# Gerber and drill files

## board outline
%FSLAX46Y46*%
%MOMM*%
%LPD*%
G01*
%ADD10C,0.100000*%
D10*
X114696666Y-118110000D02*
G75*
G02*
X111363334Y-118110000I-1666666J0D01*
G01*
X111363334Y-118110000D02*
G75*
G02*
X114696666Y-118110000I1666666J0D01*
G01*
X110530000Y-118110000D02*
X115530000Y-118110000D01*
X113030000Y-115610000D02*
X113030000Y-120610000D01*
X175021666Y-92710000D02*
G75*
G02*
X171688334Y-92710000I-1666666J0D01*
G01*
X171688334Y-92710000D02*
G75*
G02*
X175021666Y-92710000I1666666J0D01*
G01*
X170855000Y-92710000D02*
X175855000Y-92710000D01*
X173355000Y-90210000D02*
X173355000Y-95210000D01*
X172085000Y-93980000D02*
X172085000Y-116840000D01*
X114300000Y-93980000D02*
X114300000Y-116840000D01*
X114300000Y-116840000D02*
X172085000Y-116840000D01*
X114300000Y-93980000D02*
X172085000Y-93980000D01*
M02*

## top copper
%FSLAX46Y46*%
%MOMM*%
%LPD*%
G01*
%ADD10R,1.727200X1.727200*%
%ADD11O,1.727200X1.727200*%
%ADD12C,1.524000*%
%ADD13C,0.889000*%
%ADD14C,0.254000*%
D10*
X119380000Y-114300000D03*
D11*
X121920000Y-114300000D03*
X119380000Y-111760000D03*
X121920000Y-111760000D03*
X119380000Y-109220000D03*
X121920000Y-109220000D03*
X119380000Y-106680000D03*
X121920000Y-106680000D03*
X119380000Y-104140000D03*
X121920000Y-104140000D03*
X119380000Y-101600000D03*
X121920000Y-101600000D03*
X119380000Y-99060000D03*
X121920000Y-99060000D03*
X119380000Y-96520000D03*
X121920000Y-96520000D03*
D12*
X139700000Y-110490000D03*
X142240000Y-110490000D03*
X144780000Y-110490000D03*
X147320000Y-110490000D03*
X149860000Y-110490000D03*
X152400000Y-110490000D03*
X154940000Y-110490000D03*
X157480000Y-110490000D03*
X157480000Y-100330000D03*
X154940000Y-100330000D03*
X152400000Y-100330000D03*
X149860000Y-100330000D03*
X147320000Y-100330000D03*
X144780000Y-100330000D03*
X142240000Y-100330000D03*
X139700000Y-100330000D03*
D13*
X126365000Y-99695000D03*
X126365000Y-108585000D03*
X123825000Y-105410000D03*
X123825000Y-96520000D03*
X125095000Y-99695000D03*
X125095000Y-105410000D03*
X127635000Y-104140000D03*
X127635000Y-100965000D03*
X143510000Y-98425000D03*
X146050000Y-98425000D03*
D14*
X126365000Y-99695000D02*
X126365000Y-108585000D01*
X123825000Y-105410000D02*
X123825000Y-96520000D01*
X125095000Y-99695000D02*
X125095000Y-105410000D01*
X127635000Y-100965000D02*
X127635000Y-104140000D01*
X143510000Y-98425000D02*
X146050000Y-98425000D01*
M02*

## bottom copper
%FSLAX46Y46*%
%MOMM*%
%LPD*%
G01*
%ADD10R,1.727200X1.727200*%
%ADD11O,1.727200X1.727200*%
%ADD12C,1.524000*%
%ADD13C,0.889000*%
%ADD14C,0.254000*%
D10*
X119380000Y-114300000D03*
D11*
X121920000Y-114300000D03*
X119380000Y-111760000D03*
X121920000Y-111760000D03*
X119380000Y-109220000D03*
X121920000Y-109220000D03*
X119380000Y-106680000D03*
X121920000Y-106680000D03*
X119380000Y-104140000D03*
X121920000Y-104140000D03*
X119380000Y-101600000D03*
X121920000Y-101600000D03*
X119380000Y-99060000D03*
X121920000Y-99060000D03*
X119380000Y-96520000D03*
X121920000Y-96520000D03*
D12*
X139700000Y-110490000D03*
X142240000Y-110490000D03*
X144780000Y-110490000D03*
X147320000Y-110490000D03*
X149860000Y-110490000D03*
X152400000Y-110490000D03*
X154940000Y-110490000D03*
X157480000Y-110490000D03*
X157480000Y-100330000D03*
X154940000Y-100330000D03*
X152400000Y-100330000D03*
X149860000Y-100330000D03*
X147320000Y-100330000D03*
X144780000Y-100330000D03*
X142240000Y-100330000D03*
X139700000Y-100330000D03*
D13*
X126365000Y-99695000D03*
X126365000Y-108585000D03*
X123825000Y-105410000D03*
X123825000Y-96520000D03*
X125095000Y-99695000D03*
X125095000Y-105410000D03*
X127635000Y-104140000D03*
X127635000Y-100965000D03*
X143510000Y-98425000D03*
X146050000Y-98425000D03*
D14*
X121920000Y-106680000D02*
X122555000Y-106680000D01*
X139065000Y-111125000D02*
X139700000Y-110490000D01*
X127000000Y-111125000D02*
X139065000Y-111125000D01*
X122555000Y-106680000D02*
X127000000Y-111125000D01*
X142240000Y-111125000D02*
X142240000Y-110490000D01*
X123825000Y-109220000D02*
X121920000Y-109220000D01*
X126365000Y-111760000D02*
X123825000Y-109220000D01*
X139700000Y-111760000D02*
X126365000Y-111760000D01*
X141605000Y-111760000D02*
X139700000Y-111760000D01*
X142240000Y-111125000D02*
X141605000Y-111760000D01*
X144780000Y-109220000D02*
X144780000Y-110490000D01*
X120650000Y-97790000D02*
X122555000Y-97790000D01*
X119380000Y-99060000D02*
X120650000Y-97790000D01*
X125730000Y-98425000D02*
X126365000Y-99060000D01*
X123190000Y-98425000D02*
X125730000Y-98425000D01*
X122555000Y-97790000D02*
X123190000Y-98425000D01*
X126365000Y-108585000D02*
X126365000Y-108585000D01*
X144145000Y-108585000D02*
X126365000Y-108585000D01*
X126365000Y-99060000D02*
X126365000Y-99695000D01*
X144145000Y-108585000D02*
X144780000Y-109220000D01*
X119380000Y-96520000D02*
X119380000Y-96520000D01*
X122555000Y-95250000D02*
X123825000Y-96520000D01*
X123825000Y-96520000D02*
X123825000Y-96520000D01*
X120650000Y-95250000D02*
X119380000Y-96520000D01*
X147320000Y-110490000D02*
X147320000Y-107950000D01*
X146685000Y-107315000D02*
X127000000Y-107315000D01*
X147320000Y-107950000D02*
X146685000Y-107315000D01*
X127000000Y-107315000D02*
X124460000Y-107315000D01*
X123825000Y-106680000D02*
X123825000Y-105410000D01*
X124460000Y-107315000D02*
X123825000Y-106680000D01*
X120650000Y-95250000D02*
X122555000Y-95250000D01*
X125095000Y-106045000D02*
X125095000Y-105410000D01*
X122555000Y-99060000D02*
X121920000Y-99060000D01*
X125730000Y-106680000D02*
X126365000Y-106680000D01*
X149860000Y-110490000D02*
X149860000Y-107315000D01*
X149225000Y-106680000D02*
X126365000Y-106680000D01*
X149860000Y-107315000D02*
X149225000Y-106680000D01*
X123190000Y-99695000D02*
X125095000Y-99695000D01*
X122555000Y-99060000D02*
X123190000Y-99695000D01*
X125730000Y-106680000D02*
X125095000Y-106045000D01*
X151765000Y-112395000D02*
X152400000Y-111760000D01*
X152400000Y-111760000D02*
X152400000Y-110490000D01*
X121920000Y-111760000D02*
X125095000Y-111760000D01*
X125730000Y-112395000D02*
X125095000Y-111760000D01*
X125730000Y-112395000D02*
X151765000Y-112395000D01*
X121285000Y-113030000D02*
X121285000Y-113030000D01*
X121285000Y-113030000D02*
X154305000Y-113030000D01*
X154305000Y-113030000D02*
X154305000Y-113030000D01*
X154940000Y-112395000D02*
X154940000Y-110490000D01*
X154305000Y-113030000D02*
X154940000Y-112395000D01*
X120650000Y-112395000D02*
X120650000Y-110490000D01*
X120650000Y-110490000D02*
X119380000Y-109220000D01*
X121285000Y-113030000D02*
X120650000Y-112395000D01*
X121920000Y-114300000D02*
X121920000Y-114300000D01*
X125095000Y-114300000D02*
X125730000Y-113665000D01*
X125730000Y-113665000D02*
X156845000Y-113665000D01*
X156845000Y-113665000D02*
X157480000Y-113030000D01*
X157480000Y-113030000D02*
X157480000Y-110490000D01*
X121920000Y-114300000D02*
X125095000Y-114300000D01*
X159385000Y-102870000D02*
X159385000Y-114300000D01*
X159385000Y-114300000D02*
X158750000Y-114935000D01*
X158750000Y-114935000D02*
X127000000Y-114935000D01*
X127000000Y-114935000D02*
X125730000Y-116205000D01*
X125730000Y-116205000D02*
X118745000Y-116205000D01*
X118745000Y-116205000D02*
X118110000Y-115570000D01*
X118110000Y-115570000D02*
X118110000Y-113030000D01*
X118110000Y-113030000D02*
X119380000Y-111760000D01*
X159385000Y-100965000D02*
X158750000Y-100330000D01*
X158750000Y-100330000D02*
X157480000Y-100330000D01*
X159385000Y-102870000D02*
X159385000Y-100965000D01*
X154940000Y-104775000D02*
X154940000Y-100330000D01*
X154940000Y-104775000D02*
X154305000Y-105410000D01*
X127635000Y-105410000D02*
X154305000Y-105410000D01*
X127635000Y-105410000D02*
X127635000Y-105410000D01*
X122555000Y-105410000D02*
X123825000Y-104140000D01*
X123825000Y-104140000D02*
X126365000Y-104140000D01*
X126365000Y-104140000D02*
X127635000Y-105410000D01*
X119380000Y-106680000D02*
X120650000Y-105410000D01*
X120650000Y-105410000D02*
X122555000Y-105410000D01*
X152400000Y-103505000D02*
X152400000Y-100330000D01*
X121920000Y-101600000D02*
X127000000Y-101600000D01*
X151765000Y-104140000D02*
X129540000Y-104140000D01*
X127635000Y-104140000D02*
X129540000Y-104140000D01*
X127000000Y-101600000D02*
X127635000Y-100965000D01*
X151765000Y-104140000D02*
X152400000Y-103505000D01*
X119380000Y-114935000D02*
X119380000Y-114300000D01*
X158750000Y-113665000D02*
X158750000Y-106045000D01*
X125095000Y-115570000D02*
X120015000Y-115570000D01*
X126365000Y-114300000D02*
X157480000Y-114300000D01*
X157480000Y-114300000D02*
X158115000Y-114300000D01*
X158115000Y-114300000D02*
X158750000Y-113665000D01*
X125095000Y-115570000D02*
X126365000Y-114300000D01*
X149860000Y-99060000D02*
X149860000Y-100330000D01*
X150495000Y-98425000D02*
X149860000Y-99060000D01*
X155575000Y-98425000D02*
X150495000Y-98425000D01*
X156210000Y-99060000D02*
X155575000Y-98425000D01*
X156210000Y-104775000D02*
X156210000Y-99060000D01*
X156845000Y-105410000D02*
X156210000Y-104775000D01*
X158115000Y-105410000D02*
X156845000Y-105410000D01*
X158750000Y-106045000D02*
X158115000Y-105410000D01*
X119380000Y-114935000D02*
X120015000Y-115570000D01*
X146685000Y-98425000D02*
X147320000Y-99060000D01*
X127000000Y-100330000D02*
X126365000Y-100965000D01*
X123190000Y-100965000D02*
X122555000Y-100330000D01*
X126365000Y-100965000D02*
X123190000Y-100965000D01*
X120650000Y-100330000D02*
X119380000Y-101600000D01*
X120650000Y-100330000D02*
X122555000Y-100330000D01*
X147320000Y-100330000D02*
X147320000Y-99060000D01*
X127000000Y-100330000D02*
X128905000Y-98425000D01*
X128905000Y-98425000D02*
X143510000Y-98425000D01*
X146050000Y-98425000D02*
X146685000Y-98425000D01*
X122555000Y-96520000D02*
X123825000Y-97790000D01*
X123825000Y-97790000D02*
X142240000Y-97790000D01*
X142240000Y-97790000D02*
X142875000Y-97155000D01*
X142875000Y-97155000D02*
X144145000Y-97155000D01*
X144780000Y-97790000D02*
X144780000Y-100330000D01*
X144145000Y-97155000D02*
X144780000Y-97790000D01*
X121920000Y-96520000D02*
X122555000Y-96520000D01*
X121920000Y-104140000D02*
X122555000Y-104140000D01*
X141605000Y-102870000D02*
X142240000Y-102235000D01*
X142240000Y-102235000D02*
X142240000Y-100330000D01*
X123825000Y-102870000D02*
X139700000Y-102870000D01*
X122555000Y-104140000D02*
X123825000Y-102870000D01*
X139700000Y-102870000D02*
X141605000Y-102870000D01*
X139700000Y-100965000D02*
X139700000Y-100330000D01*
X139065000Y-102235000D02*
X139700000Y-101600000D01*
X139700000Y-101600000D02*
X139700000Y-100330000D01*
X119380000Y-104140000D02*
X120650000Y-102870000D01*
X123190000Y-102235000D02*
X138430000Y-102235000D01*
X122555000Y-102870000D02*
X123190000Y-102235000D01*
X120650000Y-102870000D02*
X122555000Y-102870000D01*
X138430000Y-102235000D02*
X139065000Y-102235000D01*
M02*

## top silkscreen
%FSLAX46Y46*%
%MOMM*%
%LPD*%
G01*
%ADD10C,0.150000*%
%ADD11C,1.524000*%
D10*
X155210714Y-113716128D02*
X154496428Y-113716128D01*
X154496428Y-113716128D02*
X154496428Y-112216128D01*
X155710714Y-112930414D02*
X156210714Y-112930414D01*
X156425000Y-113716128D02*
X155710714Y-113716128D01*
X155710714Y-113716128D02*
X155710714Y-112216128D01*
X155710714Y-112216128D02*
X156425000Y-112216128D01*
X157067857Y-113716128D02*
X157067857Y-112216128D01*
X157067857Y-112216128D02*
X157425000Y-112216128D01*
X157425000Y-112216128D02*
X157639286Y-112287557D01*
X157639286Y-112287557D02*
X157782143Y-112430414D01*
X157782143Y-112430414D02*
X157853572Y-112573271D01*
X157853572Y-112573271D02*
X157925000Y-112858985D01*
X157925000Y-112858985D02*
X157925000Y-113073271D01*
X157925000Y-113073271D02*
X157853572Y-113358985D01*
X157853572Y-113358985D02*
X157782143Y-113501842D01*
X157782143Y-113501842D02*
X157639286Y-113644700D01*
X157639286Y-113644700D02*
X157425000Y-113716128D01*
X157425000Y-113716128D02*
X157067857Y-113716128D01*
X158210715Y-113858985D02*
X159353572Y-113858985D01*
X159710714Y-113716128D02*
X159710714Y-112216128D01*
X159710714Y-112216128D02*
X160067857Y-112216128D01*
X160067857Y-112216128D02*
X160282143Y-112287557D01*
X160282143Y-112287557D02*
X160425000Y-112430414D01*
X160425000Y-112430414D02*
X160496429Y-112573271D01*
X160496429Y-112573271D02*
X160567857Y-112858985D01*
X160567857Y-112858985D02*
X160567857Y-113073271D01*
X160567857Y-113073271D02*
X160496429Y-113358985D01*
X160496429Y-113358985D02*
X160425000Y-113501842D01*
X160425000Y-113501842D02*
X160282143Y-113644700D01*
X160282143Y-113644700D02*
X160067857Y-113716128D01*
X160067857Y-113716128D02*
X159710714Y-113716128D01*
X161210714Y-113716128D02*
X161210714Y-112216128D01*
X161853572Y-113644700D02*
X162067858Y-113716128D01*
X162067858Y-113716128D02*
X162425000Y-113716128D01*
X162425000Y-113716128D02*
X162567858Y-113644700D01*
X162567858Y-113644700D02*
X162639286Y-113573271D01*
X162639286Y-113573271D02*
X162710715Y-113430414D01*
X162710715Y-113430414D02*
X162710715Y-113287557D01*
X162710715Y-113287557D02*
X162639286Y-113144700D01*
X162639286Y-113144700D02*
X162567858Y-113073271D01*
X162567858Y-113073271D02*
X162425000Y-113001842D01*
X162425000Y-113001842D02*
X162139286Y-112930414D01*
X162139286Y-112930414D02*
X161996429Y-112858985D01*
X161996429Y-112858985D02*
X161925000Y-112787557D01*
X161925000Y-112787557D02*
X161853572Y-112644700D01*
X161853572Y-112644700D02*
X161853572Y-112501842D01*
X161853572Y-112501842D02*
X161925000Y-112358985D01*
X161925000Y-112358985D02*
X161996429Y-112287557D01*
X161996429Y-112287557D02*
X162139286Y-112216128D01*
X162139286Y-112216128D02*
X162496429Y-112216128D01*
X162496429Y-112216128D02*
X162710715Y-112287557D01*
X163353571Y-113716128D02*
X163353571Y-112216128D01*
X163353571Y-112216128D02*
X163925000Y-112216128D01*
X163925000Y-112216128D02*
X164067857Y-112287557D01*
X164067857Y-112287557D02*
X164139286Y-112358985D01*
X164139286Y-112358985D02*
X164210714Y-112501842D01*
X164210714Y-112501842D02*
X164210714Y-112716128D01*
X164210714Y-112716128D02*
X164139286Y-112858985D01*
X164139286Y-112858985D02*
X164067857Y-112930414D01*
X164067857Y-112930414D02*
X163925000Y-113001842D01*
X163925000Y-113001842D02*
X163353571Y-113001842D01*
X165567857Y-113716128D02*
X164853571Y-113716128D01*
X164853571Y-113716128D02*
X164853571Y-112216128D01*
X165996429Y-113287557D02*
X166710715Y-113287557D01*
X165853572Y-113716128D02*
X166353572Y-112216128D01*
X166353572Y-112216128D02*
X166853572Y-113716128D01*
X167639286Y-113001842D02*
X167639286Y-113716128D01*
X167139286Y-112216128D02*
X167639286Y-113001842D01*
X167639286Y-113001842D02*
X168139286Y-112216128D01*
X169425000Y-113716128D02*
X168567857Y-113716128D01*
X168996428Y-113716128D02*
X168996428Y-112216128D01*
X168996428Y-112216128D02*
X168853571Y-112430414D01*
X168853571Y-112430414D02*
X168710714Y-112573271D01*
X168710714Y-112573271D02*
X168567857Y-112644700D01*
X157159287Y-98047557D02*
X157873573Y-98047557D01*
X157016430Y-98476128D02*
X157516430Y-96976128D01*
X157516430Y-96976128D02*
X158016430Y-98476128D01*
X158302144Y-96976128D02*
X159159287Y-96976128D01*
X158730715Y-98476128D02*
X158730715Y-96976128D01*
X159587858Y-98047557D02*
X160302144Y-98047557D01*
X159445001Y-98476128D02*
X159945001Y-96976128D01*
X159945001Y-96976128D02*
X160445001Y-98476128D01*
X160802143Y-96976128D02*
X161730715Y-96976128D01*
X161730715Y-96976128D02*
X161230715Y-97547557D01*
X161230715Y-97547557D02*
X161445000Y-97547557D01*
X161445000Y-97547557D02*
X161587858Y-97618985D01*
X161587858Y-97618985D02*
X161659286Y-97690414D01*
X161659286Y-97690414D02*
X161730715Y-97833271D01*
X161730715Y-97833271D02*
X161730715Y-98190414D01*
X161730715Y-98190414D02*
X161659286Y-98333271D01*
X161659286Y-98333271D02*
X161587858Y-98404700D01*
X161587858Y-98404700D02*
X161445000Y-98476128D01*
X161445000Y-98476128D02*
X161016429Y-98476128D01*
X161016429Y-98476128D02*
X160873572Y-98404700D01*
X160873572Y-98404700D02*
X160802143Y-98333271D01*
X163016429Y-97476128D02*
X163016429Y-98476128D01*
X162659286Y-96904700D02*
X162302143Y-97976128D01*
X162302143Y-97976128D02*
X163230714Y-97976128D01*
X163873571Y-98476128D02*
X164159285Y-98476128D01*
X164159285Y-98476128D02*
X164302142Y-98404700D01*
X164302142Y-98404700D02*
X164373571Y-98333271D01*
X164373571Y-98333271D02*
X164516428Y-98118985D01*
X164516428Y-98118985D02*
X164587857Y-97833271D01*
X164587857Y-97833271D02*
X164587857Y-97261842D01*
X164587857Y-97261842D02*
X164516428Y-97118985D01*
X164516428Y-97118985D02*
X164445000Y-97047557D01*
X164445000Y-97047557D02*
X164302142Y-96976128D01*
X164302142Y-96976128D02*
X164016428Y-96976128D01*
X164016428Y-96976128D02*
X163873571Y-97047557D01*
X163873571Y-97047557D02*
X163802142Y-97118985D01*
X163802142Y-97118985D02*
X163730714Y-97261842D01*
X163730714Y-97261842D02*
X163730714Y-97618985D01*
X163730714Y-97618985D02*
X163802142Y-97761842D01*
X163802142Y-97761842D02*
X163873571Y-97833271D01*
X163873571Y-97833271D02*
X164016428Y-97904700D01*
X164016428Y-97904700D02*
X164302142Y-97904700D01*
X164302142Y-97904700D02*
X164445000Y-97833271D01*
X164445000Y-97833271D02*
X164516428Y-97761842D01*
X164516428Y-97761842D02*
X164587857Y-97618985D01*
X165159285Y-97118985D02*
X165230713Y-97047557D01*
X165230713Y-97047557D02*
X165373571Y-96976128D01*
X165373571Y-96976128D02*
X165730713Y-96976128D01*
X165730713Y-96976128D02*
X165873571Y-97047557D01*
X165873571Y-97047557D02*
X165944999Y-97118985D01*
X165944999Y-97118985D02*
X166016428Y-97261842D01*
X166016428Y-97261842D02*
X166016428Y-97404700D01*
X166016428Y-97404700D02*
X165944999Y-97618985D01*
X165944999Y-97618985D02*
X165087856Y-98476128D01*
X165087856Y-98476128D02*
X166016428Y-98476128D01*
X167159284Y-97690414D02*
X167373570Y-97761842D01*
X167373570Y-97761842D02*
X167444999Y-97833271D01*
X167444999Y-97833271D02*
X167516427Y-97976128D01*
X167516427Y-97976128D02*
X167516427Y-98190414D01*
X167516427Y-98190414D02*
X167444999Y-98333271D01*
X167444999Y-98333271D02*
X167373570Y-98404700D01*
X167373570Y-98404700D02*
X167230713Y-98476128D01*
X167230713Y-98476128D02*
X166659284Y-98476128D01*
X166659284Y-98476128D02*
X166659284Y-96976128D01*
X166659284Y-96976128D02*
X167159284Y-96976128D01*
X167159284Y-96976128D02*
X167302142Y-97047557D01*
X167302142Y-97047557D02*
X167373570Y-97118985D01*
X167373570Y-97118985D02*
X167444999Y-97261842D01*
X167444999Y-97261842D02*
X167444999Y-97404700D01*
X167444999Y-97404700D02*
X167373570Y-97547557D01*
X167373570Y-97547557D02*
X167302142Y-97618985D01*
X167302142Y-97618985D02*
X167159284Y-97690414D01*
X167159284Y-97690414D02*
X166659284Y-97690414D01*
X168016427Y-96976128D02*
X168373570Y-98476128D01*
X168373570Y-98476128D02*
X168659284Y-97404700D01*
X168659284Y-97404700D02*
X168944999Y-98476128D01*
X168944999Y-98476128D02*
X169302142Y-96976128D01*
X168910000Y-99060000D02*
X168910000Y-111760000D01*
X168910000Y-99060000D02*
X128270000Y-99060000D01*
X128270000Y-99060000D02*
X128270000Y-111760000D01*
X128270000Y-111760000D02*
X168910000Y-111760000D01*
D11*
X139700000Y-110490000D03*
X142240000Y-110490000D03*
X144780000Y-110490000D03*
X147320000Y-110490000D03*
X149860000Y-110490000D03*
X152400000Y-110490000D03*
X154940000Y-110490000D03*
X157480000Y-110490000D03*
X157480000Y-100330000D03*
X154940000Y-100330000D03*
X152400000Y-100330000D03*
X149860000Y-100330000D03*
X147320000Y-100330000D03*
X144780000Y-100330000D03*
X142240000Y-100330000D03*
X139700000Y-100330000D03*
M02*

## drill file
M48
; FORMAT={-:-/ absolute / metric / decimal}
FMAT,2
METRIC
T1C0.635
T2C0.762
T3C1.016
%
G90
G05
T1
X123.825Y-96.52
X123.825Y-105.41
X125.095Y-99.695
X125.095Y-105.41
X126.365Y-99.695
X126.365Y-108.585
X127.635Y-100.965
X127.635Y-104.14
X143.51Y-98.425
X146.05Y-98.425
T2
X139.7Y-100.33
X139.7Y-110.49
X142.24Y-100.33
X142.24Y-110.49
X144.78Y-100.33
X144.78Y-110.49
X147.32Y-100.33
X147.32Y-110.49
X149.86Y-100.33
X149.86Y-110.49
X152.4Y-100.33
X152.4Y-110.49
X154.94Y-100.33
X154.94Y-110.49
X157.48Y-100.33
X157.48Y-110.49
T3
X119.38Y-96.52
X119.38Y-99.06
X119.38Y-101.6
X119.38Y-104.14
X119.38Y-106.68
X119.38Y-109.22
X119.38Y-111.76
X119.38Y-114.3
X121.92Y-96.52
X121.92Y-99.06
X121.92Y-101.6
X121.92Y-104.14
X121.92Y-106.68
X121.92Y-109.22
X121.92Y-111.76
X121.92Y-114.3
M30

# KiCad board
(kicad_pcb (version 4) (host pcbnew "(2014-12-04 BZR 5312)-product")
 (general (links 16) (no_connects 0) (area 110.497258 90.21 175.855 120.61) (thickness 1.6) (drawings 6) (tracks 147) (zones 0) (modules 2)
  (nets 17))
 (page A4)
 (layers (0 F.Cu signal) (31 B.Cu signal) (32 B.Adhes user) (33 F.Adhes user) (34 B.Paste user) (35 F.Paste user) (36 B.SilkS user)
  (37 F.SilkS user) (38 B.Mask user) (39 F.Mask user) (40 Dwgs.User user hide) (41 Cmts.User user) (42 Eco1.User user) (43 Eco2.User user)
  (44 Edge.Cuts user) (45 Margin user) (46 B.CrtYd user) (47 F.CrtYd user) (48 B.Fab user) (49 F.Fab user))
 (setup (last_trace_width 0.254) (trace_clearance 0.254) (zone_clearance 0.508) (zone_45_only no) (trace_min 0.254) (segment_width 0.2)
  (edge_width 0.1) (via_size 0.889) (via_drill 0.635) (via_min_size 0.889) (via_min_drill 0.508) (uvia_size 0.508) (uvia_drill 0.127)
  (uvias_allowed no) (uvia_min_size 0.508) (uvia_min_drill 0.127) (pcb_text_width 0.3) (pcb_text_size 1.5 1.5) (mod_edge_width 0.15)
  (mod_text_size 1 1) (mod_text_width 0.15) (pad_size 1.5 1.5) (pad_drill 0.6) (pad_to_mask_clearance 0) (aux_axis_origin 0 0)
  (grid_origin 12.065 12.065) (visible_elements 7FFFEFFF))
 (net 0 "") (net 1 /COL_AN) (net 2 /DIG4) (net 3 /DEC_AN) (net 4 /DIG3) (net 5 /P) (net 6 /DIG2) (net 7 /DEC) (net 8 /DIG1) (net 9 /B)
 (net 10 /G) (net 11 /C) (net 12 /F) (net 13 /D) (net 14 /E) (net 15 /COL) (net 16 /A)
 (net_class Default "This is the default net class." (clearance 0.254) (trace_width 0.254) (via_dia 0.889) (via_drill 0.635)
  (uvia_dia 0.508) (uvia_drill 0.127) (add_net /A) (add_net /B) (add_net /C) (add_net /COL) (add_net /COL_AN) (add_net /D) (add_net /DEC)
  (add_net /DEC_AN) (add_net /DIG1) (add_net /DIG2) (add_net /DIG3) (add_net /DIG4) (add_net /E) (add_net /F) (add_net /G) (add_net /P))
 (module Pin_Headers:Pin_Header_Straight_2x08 (layer B.Cu) (at 120.65 105.41 90)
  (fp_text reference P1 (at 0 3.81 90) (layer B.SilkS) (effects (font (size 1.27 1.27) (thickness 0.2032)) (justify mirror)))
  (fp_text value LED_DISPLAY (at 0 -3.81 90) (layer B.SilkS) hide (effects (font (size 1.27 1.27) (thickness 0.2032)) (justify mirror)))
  (pad 1 thru_hole rect (at -8.89 -1.27 90) (size 1.7272 1.7272) (drill 1.016) (layers *.Cu *.Mask B.SilkS) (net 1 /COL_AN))
  (pad 2 thru_hole oval (at -8.89 1.27 90) (size 1.7272 1.7272) (drill 1.016) (layers *.Cu *.Mask B.SilkS) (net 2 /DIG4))
  (pad 3 thru_hole oval (at -6.35 -1.27 90) (size 1.7272 1.7272) (drill 1.016) (layers *.Cu *.Mask B.SilkS) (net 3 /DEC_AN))
  (pad 4 thru_hole oval (at -6.35 1.27 90) (size 1.7272 1.7272) (drill 1.016) (layers *.Cu *.Mask B.SilkS) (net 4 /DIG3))
  (pad 5 thru_hole oval (at -3.81 -1.27 90) (size 1.7272 1.7272) (drill 1.016) (layers *.Cu *.Mask B.SilkS) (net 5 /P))
  (pad 6 thru_hole oval (at -3.81 1.27 90) (size 1.7272 1.7272) (drill 1.016) (layers *.Cu *.Mask B.SilkS) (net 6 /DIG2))
  (pad 7 thru_hole oval (at -1.27 -1.27 90) (size 1.7272 1.7272) (drill 1.016) (layers *.Cu *.Mask B.SilkS) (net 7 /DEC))
  (pad 8 thru_hole oval (at -1.27 1.27 90) (size 1.7272 1.7272) (drill 1.016) (layers *.Cu *.Mask B.SilkS) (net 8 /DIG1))
  (pad 9 thru_hole oval (at 1.27 -1.27 90) (size 1.7272 1.7272) (drill 1.016) (layers *.Cu *.Mask B.SilkS) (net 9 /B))
  (pad 10 thru_hole oval (at 1.27 1.27 90) (size 1.7272 1.7272) (drill 1.016) (layers *.Cu *.Mask B.SilkS) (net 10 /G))
  (pad 11 thru_hole oval (at 3.81 -1.27 90) (size 1.7272 1.7272) (drill 1.016) (layers *.Cu *.Mask B.SilkS) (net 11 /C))
  (pad 12 thru_hole oval (at 3.81 1.27 90) (size 1.7272 1.7272) (drill 1.016) (layers *.Cu *.Mask B.SilkS) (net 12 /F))
  (pad 13 thru_hole oval (at 6.35 -1.27 90) (size 1.7272 1.7272) (drill 1.016) (layers *.Cu *.Mask B.SilkS) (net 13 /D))
  (pad 14 thru_hole oval (at 6.35 1.27 90) (size 1.7272 1.7272) (drill 1.016) (layers *.Cu *.Mask B.SilkS) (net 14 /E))
  (pad 15 thru_hole oval (at 8.89 -1.27 90) (size 1.7272 1.7272) (drill 1.016) (layers *.Cu *.Mask B.SilkS) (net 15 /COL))
  (pad 16 thru_hole oval (at 8.89 1.27 90) (size 1.7272 1.7272) (drill 1.016) (layers *.Cu *.Mask B.SilkS) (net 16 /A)))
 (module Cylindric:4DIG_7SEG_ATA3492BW (layer F.Cu) (at 148.59 105.41)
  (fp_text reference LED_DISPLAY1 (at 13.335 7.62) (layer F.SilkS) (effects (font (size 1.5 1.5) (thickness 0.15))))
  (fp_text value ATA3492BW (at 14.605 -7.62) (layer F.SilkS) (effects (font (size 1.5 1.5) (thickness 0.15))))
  (fp_line (start 20.32 -6.35) (end 20.32 6.35) (layer F.SilkS) (width 0.15))
  (fp_line (start 20.32 -6.35) (end -20.32 -6.35) (layer F.SilkS) (width 0.15))
  (fp_line (start -20.32 -6.35) (end -20.32 6.35) (layer F.SilkS) (width 0.15))
  (fp_line (start -20.32 6.35) (end 20.32 6.35) (layer F.SilkS) (width 0.15))
  (pad 1 thru_hole circle (at -8.89 5.08) (size 1.524 1.524) (drill 0.762) (layers *.Cu *.Mask F.SilkS) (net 8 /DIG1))
  (pad 2 thru_hole circle (at -6.35 5.08) (size 1.524 1.524) (drill 0.762) (layers *.Cu *.Mask F.SilkS) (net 6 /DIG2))
  (pad 3 thru_hole circle (at -3.81 5.08) (size 1.524 1.524) (drill 0.762) (layers *.Cu *.Mask F.SilkS) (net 13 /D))
  (pad 4 thru_hole circle (at -1.27 5.08) (size 1.524 1.524) (drill 0.762) (layers *.Cu *.Mask F.SilkS) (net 15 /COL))
  (pad 5 thru_hole circle (at 1.27 5.08) (size 1.524 1.524) (drill 0.762) (layers *.Cu *.Mask F.SilkS) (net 14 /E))
  (pad 6 thru_hole circle (at 3.81 5.08) (size 1.524 1.524) (drill 0.762) (layers *.Cu *.Mask F.SilkS) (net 4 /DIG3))
  (pad 7 thru_hole circle (at 6.35 5.08) (size 1.524 1.524) (drill 0.762) (layers *.Cu *.Mask F.SilkS) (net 5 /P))
  (pad 8 thru_hole circle (at 8.89 5.08) (size 1.524 1.524) (drill 0.762) (layers *.Cu *.Mask F.SilkS) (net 2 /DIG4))
  (pad 9 thru_hole circle (at 8.89 -5.08) (size 1.524 1.524) (drill 0.762) (layers *.Cu *.Mask F.SilkS) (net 3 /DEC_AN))
  (pad 10 thru_hole circle (at 6.35 -5.08) (size 1.524 1.524) (drill 0.762) (layers *.Cu *.Mask F.SilkS) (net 7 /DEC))
  (pad 11 thru_hole circle (at 3.81 -5.08) (size 1.524 1.524) (drill 0.762) (layers *.Cu *.Mask F.SilkS) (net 12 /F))
  (pad 12 thru_hole circle (at 1.27 -5.08) (size 1.524 1.524) (drill 0.762) (layers *.Cu *.Mask F.SilkS) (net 1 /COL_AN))
  (pad 13 thru_hole circle (at -1.27 -5.08) (size 1.524 1.524) (drill 0.762) (layers *.Cu *.Mask F.SilkS) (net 11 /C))
  (pad 14 thru_hole circle (at -3.81 -5.08) (size 1.524 1.524) (drill 0.762) (layers *.Cu *.Mask F.SilkS) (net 16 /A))
  (pad 15 thru_hole circle (at -6.35 -5.08) (size 1.524 1.524) (drill 0.762) (layers *.Cu *.Mask F.SilkS) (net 10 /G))
  (pad 16 thru_hole circle (at -8.89 -5.08) (size 1.524 1.524) (drill 0.762) (layers *.Cu *.Mask F.SilkS) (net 9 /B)))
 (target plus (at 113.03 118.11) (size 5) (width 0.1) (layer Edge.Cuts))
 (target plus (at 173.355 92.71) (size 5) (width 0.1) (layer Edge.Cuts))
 (gr_line (start 172.085 93.98) (end 172.085 116.84) (angle 90) (layer Edge.Cuts) (width 0.1))
 (gr_line (start 114.3 93.98) (end 114.3 116.84) (angle 90) (layer Edge.Cuts) (width 0.1))
 (gr_line (start 114.3 116.84) (end 172.085 116.84) (angle 90) (layer Edge.Cuts) (width 0.1))
 (gr_line (start 114.3 93.98) (end 172.085 93.98) (angle 90) (layer Edge.Cuts) (width 0.1))
 (segment (start 121.92 106.68) (end 122.555 106.68) (width 0.254) (layer B.Cu) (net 8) (status 10))
 (segment (start 139.065 111.125) (end 139.7 110.49) (width 0.254) (layer B.Cu) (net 8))
 (segment (start 127 111.125) (end 139.065 111.125) (width 0.254) (layer B.Cu) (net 8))
 (segment (start 122.555 106.68) (end 127 111.125) (width 0.254) (layer B.Cu) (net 8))
 (segment (start 142.24 111.125) (end 142.24 110.49) (width 0.254) (layer B.Cu) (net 6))
 (segment (start 123.825 109.22) (end 121.92 109.22) (width 0.254) (layer B.Cu) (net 6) (status 20))
 (segment (start 126.365 111.76) (end 123.825 109.22) (width 0.254) (layer B.Cu) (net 6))
 (segment (start 139.7 111.76) (end 126.365 111.76) (width 0.254) (layer B.Cu) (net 6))
 (segment (start 141.605 111.76) (end 139.7 111.76) (width 0.254) (layer B.Cu) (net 6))
 (segment (start 142.24 111.125) (end 141.605 111.76) (width 0.254) (layer B.Cu) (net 6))
 (segment (start 144.78 109.22) (end 144.78 110.49) (width 0.254) (layer B.Cu) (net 13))
 (segment (start 120.65 97.79) (end 122.555 97.79) (width 0.254) (layer B.Cu) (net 13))
 (segment (start 119.38 99.06) (end 120.65 97.79) (width 0.254) (layer B.Cu) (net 13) (status 10))
 (segment (start 125.73 98.425) (end 126.365 99.06) (width 0.254) (layer B.Cu) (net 13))
 (segment (start 123.19 98.425) (end 125.73 98.425) (width 0.254) (layer B.Cu) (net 13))
 (segment (start 122.555 97.79) (end 123.19 98.425) (width 0.254) (layer B.Cu) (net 13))
 (via (at 126.365 99.695) (size 0.889) (layers F.Cu B.Cu) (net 13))
 (segment (start 126.365 99.695) (end 126.365 108.585) (width 0.254) (layer F.Cu) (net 13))
 (via (at 126.365 108.585) (size 0.889) (layers F.Cu B.Cu) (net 13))
 (segment (start 126.365 108.585) (end 126.365 108.585) (width 0.254) (layer B.Cu) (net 13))
 (segment (start 144.145 108.585) (end 126.365 108.585) (width 0.254) (layer B.Cu) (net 13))
 (segment (start 126.365 99.06) (end 126.365 99.695) (width 0.254) (layer B.Cu) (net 13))
 (segment (start 144.145 108.585) (end 144.78 109.22) (width 0.254) (layer B.Cu) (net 13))
 (segment (start 119.38 96.52) (end 119.38 96.52) (width 0.254) (layer B.Cu) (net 15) (status 30))
 (segment (start 122.555 95.25) (end 123.825 96.52) (width 0.254) (layer B.Cu) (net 15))
 (segment (start 123.825 96.52) (end 123.825 96.52) (width 0.254) (layer B.Cu) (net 15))
 (via (at 123.825 105.41) (size 0.889) (layers F.Cu B.Cu) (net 15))
 (segment (start 123.825 105.41) (end 123.825 96.52) (width 0.254) (layer F.Cu) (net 15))
 (via (at 123.825 96.52) (size 0.889) (layers F.Cu B.Cu) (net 15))
 (segment (start 120.65 95.25) (end 119.38 96.52) (width 0.254) (layer B.Cu) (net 15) (status 20))
 (segment (start 147.32 110.49) (end 147.32 107.95) (width 0.254) (layer B.Cu) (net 15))
 (segment (start 146.685 107.315) (end 127 107.315) (width 0.254) (layer B.Cu) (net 15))
 (segment (start 147.32 107.95) (end 146.685 107.315) (width 0.254) (layer B.Cu) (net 15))
 (segment (start 127 107.315) (end 124.46 107.315) (width 0.254) (layer B.Cu) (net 15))
 (segment (start 123.825 106.68) (end 123.825 105.41) (width 0.254) (layer B.Cu) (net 15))
 (segment (start 124.46 107.315) (end 123.825 106.68) (width 0.254) (layer B.Cu) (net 15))
 (segment (start 120.65 95.25) (end 122.555 95.25) (width 0.254) (layer B.Cu) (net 15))
 (segment (start 125.095 106.045) (end 125.095 105.41) (width 0.254) (layer B.Cu) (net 14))
 (segment (start 122.555 99.06) (end 121.92 99.06) (width 0.254) (layer B.Cu) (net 14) (status 20))
 (via (at 125.095 99.695) (size 0.889) (layers F.Cu B.Cu) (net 14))
 (segment (start 125.095 99.695) (end 125.095 105.41) (width 0.254) (layer F.Cu) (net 14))
 (via (at 125.095 105.41) (size 0.889) (layers F.Cu B.Cu) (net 14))
 (segment (start 125.73 106.68) (end 126.365 106.68) (width 0.254) (layer B.Cu) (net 14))
 (segment (start 149.86 110.49) (end 149.86 107.315) (width 0.254) (layer B.Cu) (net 14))
 (segment (start 149.225 106.68) (end 126.365 106.68) (width 0.254) (layer B.Cu) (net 14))
 (segment (start 149.86 107.315) (end 149.225 106.68) (width 0.254) (layer B.Cu) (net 14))
 (segment (start 123.19 99.695) (end 125.095 99.695) (width 0.254) (layer B.Cu) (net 14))
 (segment (start 122.555 99.06) (end 123.19 99.695) (width 0.254) (layer B.Cu) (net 14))
 (segment (start 125.73 106.68) (end 125.095 106.045) (width 0.254) (layer B.Cu) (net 14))
 (segment (start 151.765 112.395) (end 152.4 111.76) (width 0.254) (layer B.Cu) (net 4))
 (segment (start 152.4 111.76) (end 152.4 110.49) (width 0.254) (layer B.Cu) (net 4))
 (segment (start 121.92 111.76) (end 125.095 111.76) (width 0.254) (layer B.Cu) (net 4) (status 10))
 (segment (start 125.73 112.395) (end 125.095 111.76) (width 0.254) (layer B.Cu) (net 4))
 (segment (start 125.73 112.395) (end 151.765 112.395) (width 0.254) (layer B.Cu) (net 4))
 (segment (start 121.285 113.03) (end 121.285 113.03) (width 0.254) (layer B.Cu) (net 5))
 (segment (start 121.285 113.03) (end 154.305 113.03) (width 0.254) (layer B.Cu) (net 5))
 (segment (start 154.305 113.03) (end 154.305 113.03) (width 0.254) (layer B.Cu) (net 5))
 (segment (start 154.94 112.395) (end 154.94 110.49) (width 0.254) (layer B.Cu) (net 5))
 (segment (start 154.305 113.03) (end 154.94 112.395) (width 0.254) (layer B.Cu) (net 5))
 (segment (start 120.65 112.395) (end 120.65 110.49) (width 0.254) (layer B.Cu) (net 5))
 (segment (start 120.65 110.49) (end 119.38 109.22) (width 0.254) (layer B.Cu) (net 5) (status 10))
 (segment (start 121.285 113.03) (end 120.65 112.395) (width 0.254) (layer B.Cu) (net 5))
 (segment (start 121.92 114.3) (end 121.92 114.3) (width 0.254) (layer B.Cu) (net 2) (status 30))
 (segment (start 125.095 114.3) (end 125.73 113.665) (width 0.254) (layer B.Cu) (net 2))
 (segment (start 125.73 113.665) (end 156.845 113.665) (width 0.254) (layer B.Cu) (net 2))
 (segment (start 156.845 113.665) (end 157.48 113.03) (width 0.254) (layer B.Cu) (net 2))
 (segment (start 157.48 113.03) (end 157.48 110.49) (width 0.254) (layer B.Cu) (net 2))
 (segment (start 121.92 114.3) (end 125.095 114.3) (width 0.254) (layer B.Cu) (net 2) (status 10))
 (segment (start 159.385 102.87) (end 159.385 114.3) (width 0.254) (layer B.Cu) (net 3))
 (segment (start 159.385 114.3) (end 158.75 114.935) (width 0.254) (layer B.Cu) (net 3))
 (segment (start 158.75 114.935) (end 127 114.935) (width 0.254) (layer B.Cu) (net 3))
 (segment (start 127 114.935) (end 125.73 116.205) (width 0.254) (layer B.Cu) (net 3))
 (segment (start 125.73 116.205) (end 118.745 116.205) (width 0.254) (layer B.Cu) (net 3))
 (segment (start 118.745 116.205) (end 118.11 115.57) (width 0.254) (layer B.Cu) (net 3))
 (segment (start 118.11 115.57) (end 118.11 113.03) (width 0.254) (layer B.Cu) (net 3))
 (segment (start 118.11 113.03) (end 119.38 111.76) (width 0.254) (layer B.Cu) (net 3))
 (segment (start 159.385 100.965) (end 158.75 100.33) (width 0.254) (layer B.Cu) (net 3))
 (segment (start 158.75 100.33) (end 157.48 100.33) (width 0.254) (layer B.Cu) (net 3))
 (segment (start 159.385 102.87) (end 159.385 100.965) (width 0.254) (layer B.Cu) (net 3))
 (segment (start 154.94 104.775) (end 154.94 100.33) (width 0.254) (layer B.Cu) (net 7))
 (segment (start 154.94 104.775) (end 154.305 105.41) (width 0.254) (layer B.Cu) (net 7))
 (segment (start 127.635 105.41) (end 154.305 105.41) (width 0.254) (layer B.Cu) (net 7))
 (segment (start 127.635 105.41) (end 127.635 105.41) (width 0.254) (layer B.Cu) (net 7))
 (segment (start 122.555 105.41) (end 123.825 104.14) (width 0.254) (layer B.Cu) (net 7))
 (segment (start 123.825 104.14) (end 126.365 104.14) (width 0.254) (layer B.Cu) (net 7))
 (segment (start 126.365 104.14) (end 127.635 105.41) (width 0.254) (layer B.Cu) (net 7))
 (segment (start 119.38 106.68) (end 120.65 105.41) (width 0.254) (layer B.Cu) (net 7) (status 10))
 (segment (start 120.65 105.41) (end 122.555 105.41) (width 0.254) (layer B.Cu) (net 7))
 (segment (start 152.4 103.505) (end 152.4 100.33) (width 0.254) (layer B.Cu) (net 12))
 (segment (start 121.92 101.6) (end 127 101.6) (width 0.254) (layer B.Cu) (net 12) (status 10))
 (segment (start 151.765 104.14) (end 129.54 104.14) (width 0.254) (layer B.Cu) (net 12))
 (segment (start 127.635 104.14) (end 129.54 104.14) (width 0.254) (layer B.Cu) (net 12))
 (via (at 127.635 104.14) (size 0.889) (layers F.Cu B.Cu) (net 12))
 (segment (start 127.635 100.965) (end 127.635 104.14) (width 0.254) (layer F.Cu) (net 12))
 (via (at 127.635 100.965) (size 0.889) (layers F.Cu B.Cu) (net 12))
 (segment (start 127 101.6) (end 127.635 100.965) (width 0.254) (layer B.Cu) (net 12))
 (segment (start 151.765 104.14) (end 152.4 103.505) (width 0.254) (layer B.Cu) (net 12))
 (segment (start 119.38 114.935) (end 119.38 114.3) (width 0.254) (layer B.Cu) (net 1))
 (segment (start 158.75 113.665) (end 158.75 106.045) (width 0.254) (layer B.Cu) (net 1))
 (segment (start 125.095 115.57) (end 120.015 115.57) (width 0.254) (layer B.Cu) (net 1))
 (segment (start 126.365 114.3) (end 157.48 114.3) (width 0.254) (layer B.Cu) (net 1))
 (segment (start 157.48 114.3) (end 158.115 114.3) (width 0.254) (layer B.Cu) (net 1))
 (segment (start 158.115 114.3) (end 158.75 113.665) (width 0.254) (layer B.Cu) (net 1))
 (segment (start 125.095 115.57) (end 126.365 114.3) (width 0.254) (layer B.Cu) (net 1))
 (segment (start 149.86 99.06) (end 149.86 100.33) (width 0.254) (layer B.Cu) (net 1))
 (segment (start 150.495 98.425) (end 149.86 99.06) (width 0.254) (layer B.Cu) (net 1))
 (segment (start 155.575 98.425) (end 150.495 98.425) (width 0.254) (layer B.Cu) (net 1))
 (segment (start 156.21 99.06) (end 155.575 98.425) (width 0.254) (layer B.Cu) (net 1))
 (segment (start 156.21 104.775) (end 156.21 99.06) (width 0.254) (layer B.Cu) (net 1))
 (segment (start 156.845 105.41) (end 156.21 104.775) (width 0.254) (layer B.Cu) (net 1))
 (segment (start 158.115 105.41) (end 156.845 105.41) (width 0.254) (layer B.Cu) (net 1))
 (segment (start 158.75 106.045) (end 158.115 105.41) (width 0.254) (layer B.Cu) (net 1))
 (segment (start 119.38 114.935) (end 120.015 115.57) (width 0.254) (layer B.Cu) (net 1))
 (segment (start 146.685 98.425) (end 147.32 99.06) (width 0.254) (layer B.Cu) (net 11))
 (segment (start 127 100.33) (end 126.365 100.965) (width 0.254) (layer B.Cu) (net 11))
 (segment (start 123.19 100.965) (end 122.555 100.33) (width 0.254) (layer B.Cu) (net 11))
 (segment (start 126.365 100.965) (end 123.19 100.965) (width 0.254) (layer B.Cu) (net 11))
 (segment (start 120.65 100.33) (end 119.38 101.6) (width 0.254) (layer B.Cu) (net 11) (status 20))
 (segment (start 120.65 100.33) (end 122.555 100.33) (width 0.254) (layer B.Cu) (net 11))
 (segment (start 147.32 100.33) (end 147.32 99.06) (width 0.254) (layer B.Cu) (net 11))
 (segment (start 127 100.33) (end 128.905 98.425) (width 0.254) (layer B.Cu) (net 11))
 (segment (start 128.905 98.425) (end 143.51 98.425) (width 0.254) (layer B.Cu) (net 11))
 (via (at 143.51 98.425) (size 0.889) (layers F.Cu B.Cu) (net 11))
 (segment (start 143.51 98.425) (end 146.05 98.425) (width 0.254) (layer F.Cu) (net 11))
 (via (at 146.05 98.425) (size 0.889) (layers F.Cu B.Cu) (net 11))
 (segment (start 146.05 98.425) (end 146.685 98.425) (width 0.254) (layer B.Cu) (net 11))
 (segment (start 122.555 96.52) (end 123.825 97.79) (width 0.254) (layer B.Cu) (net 16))
 (segment (start 123.825 97.79) (end 142.24 97.79) (width 0.254) (layer B.Cu) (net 16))
 (segment (start 142.24 97.79) (end 142.875 97.155) (width 0.254) (layer B.Cu) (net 16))
 (segment (start 142.875 97.155) (end 144.145 97.155) (width 0.254) (layer B.Cu) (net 16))
 (segment (start 144.78 97.79) (end 144.78 100.33) (width 0.254) (layer B.Cu) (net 16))
 (segment (start 144.145 97.155) (end 144.78 97.79) (width 0.254) (layer B.Cu) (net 16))
 (segment (start 121.92 96.52) (end 122.555 96.52) (width 0.254) (layer B.Cu) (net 16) (status 10))
 (segment (start 121.92 104.14) (end 122.555 104.14) (width 0.254) (layer B.Cu) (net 10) (status 10))
 (segment (start 141.605 102.87) (end 142.24 102.235) (width 0.254) (layer B.Cu) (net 10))
 (segment (start 142.24 102.235) (end 142.24 100.33) (width 0.254) (layer B.Cu) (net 10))
 (segment (start 123.825 102.87) (end 139.7 102.87) (width 0.254) (layer B.Cu) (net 10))
 (segment (start 122.555 104.14) (end 123.825 102.87) (width 0.254) (layer B.Cu) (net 10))
 (segment (start 139.7 102.87) (end 141.605 102.87) (width 0.254) (layer B.Cu) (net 10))
 (segment (start 139.7 100.965) (end 139.7 100.33) (width 0.254) (layer B.Cu) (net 9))
 (segment (start 139.065 102.235) (end 139.7 101.6) (width 0.254) (layer B.Cu) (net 9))
 (segment (start 139.7 101.6) (end 139.7 100.33) (width 0.254) (layer B.Cu) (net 9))
 (segment (start 119.38 104.14) (end 120.65 102.87) (width 0.254) (layer B.Cu) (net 9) (status 10))
 (segment (start 123.19 102.235) (end 138.43 102.235) (width 0.254) (layer B.Cu) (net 9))
 (segment (start 122.555 102.87) (end 123.19 102.235) (width 0.254) (layer B.Cu) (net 9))
 (segment (start 120.65 102.87) (end 122.555 102.87) (width 0.254) (layer B.Cu) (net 9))
 (segment (start 138.43 102.235) (end 139.065 102.235) (width 0.254) (layer B.Cu) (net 9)))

